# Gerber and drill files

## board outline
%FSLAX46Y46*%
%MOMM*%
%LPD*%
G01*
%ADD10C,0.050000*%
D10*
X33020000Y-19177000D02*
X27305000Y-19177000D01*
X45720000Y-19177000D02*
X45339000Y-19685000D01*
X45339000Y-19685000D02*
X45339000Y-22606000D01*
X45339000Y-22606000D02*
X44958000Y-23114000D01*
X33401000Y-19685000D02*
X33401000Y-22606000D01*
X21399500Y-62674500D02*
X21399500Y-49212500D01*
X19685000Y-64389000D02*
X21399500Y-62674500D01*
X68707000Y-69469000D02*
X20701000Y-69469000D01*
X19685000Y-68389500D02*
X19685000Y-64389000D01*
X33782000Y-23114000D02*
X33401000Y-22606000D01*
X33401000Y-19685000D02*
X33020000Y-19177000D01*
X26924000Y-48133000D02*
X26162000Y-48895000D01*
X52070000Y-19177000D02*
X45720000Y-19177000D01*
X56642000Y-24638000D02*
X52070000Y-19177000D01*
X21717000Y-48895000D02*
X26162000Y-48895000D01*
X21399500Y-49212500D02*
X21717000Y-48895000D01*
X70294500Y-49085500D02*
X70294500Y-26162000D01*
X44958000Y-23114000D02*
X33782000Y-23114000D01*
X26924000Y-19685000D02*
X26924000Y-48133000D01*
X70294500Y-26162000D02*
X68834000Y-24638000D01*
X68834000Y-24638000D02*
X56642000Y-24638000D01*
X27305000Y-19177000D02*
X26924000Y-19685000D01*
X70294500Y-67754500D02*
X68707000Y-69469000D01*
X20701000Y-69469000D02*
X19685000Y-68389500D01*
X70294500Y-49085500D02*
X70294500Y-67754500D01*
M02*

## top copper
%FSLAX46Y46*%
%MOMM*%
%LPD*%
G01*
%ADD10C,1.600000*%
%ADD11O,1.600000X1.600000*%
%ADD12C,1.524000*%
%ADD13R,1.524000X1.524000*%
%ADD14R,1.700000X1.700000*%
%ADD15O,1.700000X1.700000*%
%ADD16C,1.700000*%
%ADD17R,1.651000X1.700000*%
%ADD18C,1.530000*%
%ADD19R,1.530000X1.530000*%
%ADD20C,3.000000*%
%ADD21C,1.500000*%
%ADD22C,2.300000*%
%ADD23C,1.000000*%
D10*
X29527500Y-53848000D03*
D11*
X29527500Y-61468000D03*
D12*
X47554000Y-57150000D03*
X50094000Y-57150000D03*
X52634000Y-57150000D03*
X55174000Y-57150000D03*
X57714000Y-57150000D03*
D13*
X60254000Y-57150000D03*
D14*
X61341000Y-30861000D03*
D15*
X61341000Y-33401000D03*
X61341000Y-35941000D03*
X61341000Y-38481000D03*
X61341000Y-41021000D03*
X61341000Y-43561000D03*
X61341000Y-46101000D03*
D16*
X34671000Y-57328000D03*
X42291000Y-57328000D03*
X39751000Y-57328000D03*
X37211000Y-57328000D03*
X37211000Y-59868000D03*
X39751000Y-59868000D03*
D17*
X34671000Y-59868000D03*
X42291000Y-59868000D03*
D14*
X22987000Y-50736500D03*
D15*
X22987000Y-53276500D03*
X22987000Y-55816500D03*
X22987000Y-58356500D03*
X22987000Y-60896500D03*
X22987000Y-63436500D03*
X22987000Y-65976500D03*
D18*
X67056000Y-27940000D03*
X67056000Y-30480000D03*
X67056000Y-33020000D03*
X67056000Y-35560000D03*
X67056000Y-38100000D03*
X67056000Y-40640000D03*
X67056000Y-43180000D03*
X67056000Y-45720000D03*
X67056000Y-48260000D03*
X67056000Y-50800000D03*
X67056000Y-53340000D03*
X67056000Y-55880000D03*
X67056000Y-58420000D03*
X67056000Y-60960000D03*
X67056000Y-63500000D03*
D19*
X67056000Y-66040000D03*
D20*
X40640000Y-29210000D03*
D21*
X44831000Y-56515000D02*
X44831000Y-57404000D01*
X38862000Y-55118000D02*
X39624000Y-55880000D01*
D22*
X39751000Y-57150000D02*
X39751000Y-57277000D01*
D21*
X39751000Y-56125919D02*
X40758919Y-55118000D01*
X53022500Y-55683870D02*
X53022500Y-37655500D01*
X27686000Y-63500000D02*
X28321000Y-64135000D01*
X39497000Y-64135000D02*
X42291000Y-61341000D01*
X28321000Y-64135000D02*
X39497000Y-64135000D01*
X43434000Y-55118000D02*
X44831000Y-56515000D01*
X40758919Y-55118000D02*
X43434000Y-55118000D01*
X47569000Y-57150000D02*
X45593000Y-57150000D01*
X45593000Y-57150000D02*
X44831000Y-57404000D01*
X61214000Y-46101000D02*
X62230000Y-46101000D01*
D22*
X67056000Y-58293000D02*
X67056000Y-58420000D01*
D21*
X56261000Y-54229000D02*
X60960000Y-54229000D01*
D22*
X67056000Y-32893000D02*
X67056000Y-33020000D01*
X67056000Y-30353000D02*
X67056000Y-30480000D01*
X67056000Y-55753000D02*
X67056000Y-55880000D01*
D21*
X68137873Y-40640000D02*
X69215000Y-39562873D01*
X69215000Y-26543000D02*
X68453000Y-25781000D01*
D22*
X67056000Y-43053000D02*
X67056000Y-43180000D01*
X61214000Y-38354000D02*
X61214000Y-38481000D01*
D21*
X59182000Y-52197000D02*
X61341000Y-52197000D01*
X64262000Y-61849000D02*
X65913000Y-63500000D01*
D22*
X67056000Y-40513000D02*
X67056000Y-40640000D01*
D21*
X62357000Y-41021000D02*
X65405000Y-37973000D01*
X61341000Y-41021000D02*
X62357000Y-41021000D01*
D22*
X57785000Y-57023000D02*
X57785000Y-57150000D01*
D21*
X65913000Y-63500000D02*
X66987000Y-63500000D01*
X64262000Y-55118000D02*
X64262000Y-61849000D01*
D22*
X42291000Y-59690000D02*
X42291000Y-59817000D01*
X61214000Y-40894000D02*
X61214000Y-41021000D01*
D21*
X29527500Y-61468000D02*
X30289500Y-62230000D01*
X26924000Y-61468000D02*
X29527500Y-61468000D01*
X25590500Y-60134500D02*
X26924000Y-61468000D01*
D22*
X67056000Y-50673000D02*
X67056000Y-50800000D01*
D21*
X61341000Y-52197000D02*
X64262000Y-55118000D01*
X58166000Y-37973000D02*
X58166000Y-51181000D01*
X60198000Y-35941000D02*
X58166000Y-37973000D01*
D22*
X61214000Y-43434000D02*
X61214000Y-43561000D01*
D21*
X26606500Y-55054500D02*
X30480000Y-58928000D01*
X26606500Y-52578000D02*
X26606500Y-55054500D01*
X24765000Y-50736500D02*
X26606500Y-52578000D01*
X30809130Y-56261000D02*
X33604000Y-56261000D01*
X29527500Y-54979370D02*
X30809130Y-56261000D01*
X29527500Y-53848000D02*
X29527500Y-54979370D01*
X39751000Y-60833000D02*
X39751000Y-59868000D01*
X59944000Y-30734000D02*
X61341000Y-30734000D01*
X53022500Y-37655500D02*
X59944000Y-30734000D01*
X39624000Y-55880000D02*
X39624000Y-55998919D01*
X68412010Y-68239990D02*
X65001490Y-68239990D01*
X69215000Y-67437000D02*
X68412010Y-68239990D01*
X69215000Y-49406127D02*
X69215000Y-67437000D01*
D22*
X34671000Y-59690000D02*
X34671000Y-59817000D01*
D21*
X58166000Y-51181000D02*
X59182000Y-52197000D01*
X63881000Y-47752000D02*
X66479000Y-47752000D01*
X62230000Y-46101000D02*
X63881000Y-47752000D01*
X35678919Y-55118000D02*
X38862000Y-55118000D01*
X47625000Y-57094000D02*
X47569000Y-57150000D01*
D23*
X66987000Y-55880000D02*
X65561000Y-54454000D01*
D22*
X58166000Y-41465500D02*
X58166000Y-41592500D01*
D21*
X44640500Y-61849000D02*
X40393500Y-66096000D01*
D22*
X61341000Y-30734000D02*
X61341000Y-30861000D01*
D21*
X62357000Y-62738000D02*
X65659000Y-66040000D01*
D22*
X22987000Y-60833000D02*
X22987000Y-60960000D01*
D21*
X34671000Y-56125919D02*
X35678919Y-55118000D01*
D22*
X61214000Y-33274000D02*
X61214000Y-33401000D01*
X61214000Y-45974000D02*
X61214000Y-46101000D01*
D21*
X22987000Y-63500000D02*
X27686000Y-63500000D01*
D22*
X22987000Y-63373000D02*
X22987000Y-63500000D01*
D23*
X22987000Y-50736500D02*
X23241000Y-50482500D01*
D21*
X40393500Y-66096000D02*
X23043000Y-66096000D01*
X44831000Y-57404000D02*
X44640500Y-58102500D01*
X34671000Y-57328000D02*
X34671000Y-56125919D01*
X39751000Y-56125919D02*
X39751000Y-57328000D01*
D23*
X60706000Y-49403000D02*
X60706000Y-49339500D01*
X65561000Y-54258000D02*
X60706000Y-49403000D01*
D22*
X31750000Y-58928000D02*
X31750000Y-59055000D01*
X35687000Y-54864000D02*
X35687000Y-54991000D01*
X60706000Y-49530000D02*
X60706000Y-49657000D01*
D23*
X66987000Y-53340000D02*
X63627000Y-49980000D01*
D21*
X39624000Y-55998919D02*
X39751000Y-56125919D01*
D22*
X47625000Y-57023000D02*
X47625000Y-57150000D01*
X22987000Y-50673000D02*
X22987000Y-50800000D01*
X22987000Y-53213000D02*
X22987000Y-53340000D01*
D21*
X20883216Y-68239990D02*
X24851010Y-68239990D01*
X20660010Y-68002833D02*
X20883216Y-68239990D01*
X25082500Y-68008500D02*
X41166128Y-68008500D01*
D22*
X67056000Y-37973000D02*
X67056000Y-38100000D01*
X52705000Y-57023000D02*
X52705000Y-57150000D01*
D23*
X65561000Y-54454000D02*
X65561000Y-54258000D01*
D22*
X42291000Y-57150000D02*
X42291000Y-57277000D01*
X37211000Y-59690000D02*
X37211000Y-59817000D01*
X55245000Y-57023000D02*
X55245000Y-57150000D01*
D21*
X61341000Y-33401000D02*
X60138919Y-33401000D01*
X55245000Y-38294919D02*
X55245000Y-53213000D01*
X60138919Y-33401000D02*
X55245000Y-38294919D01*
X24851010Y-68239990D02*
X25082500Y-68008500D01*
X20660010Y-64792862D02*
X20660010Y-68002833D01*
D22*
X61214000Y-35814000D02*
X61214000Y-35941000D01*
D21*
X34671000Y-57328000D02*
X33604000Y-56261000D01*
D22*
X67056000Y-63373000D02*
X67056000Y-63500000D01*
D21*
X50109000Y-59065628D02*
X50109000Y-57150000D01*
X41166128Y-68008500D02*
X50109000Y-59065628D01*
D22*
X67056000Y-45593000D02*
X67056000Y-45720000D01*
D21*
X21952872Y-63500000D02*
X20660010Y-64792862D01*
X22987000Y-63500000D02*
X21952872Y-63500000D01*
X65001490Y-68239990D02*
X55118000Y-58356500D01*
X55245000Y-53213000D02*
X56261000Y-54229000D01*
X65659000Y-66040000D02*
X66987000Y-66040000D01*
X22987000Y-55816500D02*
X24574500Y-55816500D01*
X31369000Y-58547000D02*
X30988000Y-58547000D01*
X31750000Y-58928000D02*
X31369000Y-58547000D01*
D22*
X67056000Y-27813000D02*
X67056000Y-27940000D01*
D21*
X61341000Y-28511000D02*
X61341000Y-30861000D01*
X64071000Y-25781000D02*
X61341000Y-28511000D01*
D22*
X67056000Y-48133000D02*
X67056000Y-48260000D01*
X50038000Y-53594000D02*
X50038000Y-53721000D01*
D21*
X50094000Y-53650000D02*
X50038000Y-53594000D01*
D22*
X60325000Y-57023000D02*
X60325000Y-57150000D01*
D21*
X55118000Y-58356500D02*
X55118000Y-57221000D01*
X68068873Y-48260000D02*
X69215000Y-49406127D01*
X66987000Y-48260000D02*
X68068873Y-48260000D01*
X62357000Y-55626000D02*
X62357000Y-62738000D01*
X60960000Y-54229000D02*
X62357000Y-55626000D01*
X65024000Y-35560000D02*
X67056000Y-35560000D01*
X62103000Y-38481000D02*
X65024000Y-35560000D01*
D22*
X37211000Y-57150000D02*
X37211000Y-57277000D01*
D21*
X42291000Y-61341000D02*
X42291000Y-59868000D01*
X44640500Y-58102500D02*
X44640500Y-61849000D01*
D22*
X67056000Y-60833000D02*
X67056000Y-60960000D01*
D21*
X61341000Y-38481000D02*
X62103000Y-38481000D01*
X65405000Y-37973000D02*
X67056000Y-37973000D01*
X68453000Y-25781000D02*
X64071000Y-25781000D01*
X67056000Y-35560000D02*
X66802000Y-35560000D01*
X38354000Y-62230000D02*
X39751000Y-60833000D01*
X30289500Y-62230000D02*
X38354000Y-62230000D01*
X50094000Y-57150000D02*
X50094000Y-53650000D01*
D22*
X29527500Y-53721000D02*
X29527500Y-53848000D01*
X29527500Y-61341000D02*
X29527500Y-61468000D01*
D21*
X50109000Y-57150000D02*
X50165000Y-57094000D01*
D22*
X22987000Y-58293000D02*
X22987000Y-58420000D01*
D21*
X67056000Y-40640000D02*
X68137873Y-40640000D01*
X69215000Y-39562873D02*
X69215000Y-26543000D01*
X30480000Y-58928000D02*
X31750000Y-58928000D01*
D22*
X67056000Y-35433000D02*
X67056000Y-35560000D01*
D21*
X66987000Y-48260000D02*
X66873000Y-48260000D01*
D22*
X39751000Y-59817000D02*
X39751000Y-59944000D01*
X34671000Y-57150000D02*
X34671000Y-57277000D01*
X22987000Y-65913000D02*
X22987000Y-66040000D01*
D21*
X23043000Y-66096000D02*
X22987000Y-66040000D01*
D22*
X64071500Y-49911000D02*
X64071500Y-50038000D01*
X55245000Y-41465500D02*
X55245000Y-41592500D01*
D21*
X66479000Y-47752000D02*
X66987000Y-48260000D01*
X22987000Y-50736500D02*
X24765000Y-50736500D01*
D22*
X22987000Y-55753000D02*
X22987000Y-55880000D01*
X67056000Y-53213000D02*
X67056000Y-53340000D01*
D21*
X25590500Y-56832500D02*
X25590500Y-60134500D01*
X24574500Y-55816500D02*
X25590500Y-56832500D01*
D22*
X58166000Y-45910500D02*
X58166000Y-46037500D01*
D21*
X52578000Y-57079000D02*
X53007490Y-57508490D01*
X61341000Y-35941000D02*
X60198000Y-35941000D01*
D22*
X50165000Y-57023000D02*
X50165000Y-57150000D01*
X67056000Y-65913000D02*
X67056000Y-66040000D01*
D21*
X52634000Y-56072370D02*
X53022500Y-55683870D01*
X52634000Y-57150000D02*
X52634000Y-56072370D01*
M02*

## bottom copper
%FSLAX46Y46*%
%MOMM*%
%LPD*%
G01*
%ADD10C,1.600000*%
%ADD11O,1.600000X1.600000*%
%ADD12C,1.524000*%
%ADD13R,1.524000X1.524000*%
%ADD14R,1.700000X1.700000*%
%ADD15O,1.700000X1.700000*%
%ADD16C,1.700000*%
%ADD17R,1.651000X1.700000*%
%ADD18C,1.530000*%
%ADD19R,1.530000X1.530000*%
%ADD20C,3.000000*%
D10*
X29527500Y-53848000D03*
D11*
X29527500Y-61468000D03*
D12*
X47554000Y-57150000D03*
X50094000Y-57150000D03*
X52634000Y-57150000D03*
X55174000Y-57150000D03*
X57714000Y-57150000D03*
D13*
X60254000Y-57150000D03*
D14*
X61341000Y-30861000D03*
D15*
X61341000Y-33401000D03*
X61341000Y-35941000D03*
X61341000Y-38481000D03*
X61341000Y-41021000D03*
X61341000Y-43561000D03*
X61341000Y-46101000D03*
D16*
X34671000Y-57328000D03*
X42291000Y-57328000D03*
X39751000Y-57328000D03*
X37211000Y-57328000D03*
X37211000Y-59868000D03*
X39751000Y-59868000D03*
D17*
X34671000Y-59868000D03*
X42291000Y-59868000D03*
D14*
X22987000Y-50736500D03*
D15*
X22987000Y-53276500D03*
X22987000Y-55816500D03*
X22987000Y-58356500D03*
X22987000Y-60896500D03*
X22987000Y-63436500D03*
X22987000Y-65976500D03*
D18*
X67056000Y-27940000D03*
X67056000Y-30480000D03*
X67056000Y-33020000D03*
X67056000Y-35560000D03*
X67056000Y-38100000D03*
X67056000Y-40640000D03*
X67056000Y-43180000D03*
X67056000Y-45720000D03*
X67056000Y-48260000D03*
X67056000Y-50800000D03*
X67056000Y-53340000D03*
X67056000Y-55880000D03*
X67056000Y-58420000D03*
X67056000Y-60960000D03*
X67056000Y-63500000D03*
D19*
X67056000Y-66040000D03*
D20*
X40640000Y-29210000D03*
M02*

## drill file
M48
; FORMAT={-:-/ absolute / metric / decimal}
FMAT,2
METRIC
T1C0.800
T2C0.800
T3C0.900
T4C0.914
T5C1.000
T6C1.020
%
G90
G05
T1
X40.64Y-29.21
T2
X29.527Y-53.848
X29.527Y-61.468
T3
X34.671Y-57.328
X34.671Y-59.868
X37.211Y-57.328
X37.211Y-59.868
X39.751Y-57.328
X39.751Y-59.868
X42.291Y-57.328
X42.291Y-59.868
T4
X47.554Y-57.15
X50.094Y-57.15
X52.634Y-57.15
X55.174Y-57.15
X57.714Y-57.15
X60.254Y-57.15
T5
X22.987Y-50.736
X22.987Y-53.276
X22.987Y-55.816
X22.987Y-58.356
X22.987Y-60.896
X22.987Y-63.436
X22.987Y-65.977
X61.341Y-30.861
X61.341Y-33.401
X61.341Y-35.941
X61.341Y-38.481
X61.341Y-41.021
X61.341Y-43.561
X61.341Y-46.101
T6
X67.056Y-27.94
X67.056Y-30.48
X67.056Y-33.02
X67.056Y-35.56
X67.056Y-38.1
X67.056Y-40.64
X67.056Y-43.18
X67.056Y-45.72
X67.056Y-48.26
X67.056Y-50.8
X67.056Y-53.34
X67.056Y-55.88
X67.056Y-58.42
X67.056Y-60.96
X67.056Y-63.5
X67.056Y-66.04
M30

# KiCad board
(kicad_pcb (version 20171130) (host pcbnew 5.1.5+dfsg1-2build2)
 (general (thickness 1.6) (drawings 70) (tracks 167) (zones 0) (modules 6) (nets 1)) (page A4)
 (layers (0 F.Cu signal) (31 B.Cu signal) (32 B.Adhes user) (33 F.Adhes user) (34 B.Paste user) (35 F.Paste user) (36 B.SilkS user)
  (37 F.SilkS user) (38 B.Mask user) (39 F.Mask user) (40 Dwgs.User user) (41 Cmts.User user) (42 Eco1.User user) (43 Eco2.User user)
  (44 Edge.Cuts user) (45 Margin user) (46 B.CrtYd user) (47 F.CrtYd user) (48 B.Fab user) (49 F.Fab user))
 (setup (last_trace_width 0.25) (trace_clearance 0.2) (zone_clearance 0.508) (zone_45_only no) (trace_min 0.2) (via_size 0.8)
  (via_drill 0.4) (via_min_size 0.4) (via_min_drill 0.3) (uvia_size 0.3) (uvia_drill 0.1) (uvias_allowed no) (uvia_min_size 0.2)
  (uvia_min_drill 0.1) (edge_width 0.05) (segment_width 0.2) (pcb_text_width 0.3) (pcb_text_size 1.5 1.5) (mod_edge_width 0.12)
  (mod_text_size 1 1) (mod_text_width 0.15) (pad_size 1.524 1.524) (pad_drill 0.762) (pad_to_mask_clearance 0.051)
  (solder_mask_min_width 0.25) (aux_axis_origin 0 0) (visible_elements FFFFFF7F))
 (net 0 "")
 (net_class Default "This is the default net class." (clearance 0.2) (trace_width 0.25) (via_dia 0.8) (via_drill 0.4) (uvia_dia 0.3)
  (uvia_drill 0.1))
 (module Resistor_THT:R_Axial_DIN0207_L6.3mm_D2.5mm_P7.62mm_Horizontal (layer F.Cu) (at 29.5275 53.848 270)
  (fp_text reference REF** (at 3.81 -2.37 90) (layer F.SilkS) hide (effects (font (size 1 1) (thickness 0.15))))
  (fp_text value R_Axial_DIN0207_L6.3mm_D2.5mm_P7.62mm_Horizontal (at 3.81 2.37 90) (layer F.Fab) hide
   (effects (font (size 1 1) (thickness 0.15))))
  (pad 1 thru_hole circle (at 0 0 270) (size 1.6 1.6) (drill 0.8) (layers *.Cu *.Mask))
  (pad 2 thru_hole oval (at 7.62 0 270) (size 1.6 1.6) (drill 0.8) (layers *.Cu *.Mask)))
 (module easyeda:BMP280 (layer F.Cu) (at 53.721 61.468 270)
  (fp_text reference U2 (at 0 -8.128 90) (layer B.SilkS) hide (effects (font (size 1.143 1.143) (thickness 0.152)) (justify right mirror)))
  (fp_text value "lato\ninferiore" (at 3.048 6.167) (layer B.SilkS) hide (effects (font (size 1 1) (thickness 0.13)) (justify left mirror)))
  (pad 6 thru_hole circle (at -4.318 6.167 270) (size 1.524 1.524) (drill 0.914) (layers *.Cu *.Paste *.Mask))
  (pad 5 thru_hole circle (at -4.318 3.627) (size 1.524 1.524) (drill 0.914) (layers *.Cu *.Paste *.Mask))
  (pad 4 thru_hole circle (at -4.318 1.087) (size 1.524 1.524) (drill 0.914) (layers *.Cu *.Paste *.Mask))
  (pad 3 thru_hole circle (at -4.318 -1.453) (size 1.524 1.524) (drill 0.914) (layers *.Cu *.Paste *.Mask))
  (pad 2 thru_hole circle (at -4.318 -3.993) (size 1.524 1.524) (drill 0.914) (layers *.Cu *.Paste *.Mask))
  (pad 1 thru_hole rect (at -4.318 -6.533) (size 1.524 1.524) (drill 0.914) (layers *.Cu *.Paste *.Mask)))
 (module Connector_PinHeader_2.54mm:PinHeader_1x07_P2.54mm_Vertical (layer F.Cu) (at 61.341 30.861)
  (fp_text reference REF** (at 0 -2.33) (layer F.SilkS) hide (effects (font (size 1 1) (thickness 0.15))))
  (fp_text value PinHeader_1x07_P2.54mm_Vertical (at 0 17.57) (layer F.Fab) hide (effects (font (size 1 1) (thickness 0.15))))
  (pad 1 thru_hole rect (at 0 0) (size 1.7 1.7) (drill 1) (layers *.Cu *.Mask))
  (pad 2 thru_hole oval (at 0 2.54) (size 1.7 1.7) (drill 1) (layers *.Cu *.Mask))
  (pad 3 thru_hole oval (at 0 5.08) (size 1.7 1.7) (drill 1) (layers *.Cu *.Mask))
  (pad 4 thru_hole oval (at 0 7.62) (size 1.7 1.7) (drill 1) (layers *.Cu *.Mask))
  (pad 5 thru_hole oval (at 0 10.16) (size 1.7 1.7) (drill 1) (layers *.Cu *.Mask))
  (pad 6 thru_hole oval (at 0 12.7) (size 1.7 1.7) (drill 1) (layers *.Cu *.Mask))
  (pad 7 thru_hole oval (at 0 15.24) (size 1.7 1.7) (drill 1) (layers *.Cu *.Mask)))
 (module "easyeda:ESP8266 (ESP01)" (layer F.Cu) (at 45.466 80.518 180)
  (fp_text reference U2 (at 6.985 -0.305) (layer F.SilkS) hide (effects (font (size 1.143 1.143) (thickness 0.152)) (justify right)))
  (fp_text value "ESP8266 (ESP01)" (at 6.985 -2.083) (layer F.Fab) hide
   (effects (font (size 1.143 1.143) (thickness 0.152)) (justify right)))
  (pad VCC thru_hole circle (at 10.795 23.19 90) (size 1.7 1.7) (drill 0.9) (layers *.Cu *.Paste *.Mask))
  (pad TX thru_hole circle (at 3.175 23.19 90) (size 1.7 1.7) (drill 0.9) (layers *.Cu *.Paste *.Mask))
  (pad CH_PD thru_hole circle (at 5.715 23.19 90) (size 1.7 1.7) (drill 0.9) (layers *.Cu *.Paste *.Mask))
  (pad RST thru_hole circle (at 8.255 23.19 90) (size 1.7 1.7) (drill 0.9) (layers *.Cu *.Paste *.Mask))
  (pad GPIO0 thru_hole circle (at 8.255 20.65 90) (size 1.7 1.7) (drill 0.9) (layers *.Cu *.Paste *.Mask))
  (pad GPIO2 thru_hole circle (at 5.715 20.65 90) (size 1.7 1.7) (drill 0.9) (layers *.Cu *.Paste *.Mask))
  (pad RX thru_hole rect (at 10.795 20.65 90) (size 1.7 1.651) (drill 0.9) (layers *.Cu *.Paste *.Mask))
  (pad GND thru_hole rect (at 3.175 20.65 90) (size 1.7 1.651) (drill 0.9) (layers *.Cu *.Paste *.Mask)))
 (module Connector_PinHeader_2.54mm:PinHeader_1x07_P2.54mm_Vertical (layer F.Cu) (at 22.987 50.7365)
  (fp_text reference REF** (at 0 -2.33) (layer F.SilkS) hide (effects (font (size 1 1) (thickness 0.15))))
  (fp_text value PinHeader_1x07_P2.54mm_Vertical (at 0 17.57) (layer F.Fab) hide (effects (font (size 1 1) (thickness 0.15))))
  (pad 1 thru_hole rect (at 0 0) (size 1.7 1.7) (drill 1) (layers *.Cu *.Mask))
  (pad 2 thru_hole oval (at 0 2.54) (size 1.7 1.7) (drill 1) (layers *.Cu *.Mask))
  (pad 3 thru_hole oval (at 0 5.08) (size 1.7 1.7) (drill 1) (layers *.Cu *.Mask))
  (pad 4 thru_hole oval (at 0 7.62) (size 1.7 1.7) (drill 1) (layers *.Cu *.Mask))
  (pad 5 thru_hole oval (at 0 10.16) (size 1.7 1.7) (drill 1) (layers *.Cu *.Mask))
  (pad 6 thru_hole oval (at 0 12.7) (size 1.7 1.7) (drill 1) (layers *.Cu *.Mask))
  (pad 7 thru_hole oval (at 0 15.24) (size 1.7 1.7) (drill 1) (layers *.Cu *.Mask)))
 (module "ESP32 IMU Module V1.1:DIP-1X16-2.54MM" (layer F.Cu) (at 67.056 46.99 90)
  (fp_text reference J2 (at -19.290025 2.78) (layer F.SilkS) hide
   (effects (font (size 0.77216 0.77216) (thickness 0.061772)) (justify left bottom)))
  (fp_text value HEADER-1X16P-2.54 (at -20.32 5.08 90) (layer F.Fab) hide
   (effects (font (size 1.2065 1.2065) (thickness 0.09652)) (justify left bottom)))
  (pad 16 thru_hole circle (at 19.05 0 90) (size 1.53 1.53) (drill 1.02) (layers *.Cu *.Mask) (solder_mask_margin 0.1016))
  (pad 15 thru_hole circle (at 16.51 0 90) (size 1.53 1.53) (drill 1.02) (layers *.Cu *.Mask) (solder_mask_margin 0.1016))
  (pad 14 thru_hole circle (at 13.97 0 90) (size 1.53 1.53) (drill 1.02) (layers *.Cu *.Mask) (solder_mask_margin 0.1016))
  (pad 13 thru_hole circle (at 11.43 0 90) (size 1.53 1.53) (drill 1.02) (layers *.Cu *.Mask) (solder_mask_margin 0.1016))
  (pad 12 thru_hole circle (at 8.89 0 90) (size 1.53 1.53) (drill 1.02) (layers *.Cu *.Mask) (solder_mask_margin 0.1016))
  (pad 11 thru_hole circle (at 6.35 0 90) (size 1.53 1.53) (drill 1.02) (layers *.Cu *.Mask) (solder_mask_margin 0.1016))
  (pad 10 thru_hole circle (at 3.81 0 90) (size 1.53 1.53) (drill 1.02) (layers *.Cu *.Mask) (solder_mask_margin 0.1016))
  (pad 9 thru_hole circle (at 1.27 0 90) (size 1.53 1.53) (drill 1.02) (layers *.Cu *.Mask) (solder_mask_margin 0.1016))
  (pad 8 thru_hole circle (at -1.27 0 90) (size 1.53 1.53) (drill 1.02) (layers *.Cu *.Mask) (solder_mask_margin 0.1016))
  (pad 7 thru_hole circle (at -3.81 0 90) (size 1.53 1.53) (drill 1.02) (layers *.Cu *.Mask) (solder_mask_margin 0.1016))
  (pad 6 thru_hole circle (at -6.35 0 90) (size 1.53 1.53) (drill 1.02) (layers *.Cu *.Mask) (solder_mask_margin 0.1016))
  (pad 5 thru_hole circle (at -8.89 0 90) (size 1.53 1.53) (drill 1.02) (layers *.Cu *.Mask) (solder_mask_margin 0.1016))
  (pad 4 thru_hole circle (at -11.43 0 90) (size 1.53 1.53) (drill 1.02) (layers *.Cu *.Mask) (solder_mask_margin 0.1016))
  (pad 3 thru_hole circle (at -13.97 0 90) (size 1.53 1.53) (drill 1.02) (layers *.Cu *.Mask) (solder_mask_margin 0.1016))
  (pad 2 thru_hole circle (at -16.51 0 90) (size 1.53 1.53) (drill 1.02) (layers *.Cu *.Mask) (solder_mask_margin 0.1016))
  (pad 1 thru_hole rect (at -19.05 0 90) (size 1.53 1.53) (drill 1.02) (layers *.Cu *.Mask) (solder_mask_margin 0.1016)))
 (gr_line (start 33.02 19.177) (end 27.305 19.177) (layer Edge.Cuts) (width 0.05))
 (gr_line (start 45.72 19.177) (end 45.339 19.685) (layer Edge.Cuts) (width 0.05))
 (gr_line (start 45.339 19.685) (end 45.339 22.606) (layer Edge.Cuts) (width 0.05))
 (gr_line (start 45.339 22.606) (end 44.958 23.114) (layer Edge.Cuts) (width 0.05))
 (gr_line (start 33.401 19.685) (end 33.401 22.606) (layer Edge.Cuts) (width 0.05))
 (gr_line (start 21.3995 62.6745) (end 21.3995 49.2125) (layer Edge.Cuts) (width 0.05))
 (gr_line (start 19.685 64.389) (end 21.3995 62.6745) (layer Edge.Cuts) (width 0.05))
 (gr_line (start 68.707 69.469) (end 20.701 69.469) (layer Edge.Cuts) (width 0.05))
 (gr_line (start 19.685 68.3895) (end 19.685 64.389) (layer Edge.Cuts) (width 0.05))
 (gr_line (start 33.782 23.114) (end 33.401 22.606) (layer Edge.Cuts) (width 0.05))
 (gr_line (start 33.401 19.685) (end 33.02 19.177) (layer Edge.Cuts) (width 0.05))
 (gr_line (start 26.924 48.133) (end 26.162 48.895) (layer Edge.Cuts) (width 0.05))
 (gr_line (start 52.07 19.177) (end 45.72 19.177) (layer Edge.Cuts) (width 0.05))
 (gr_line (start 56.642 24.638) (end 52.07 19.177) (layer Edge.Cuts) (width 0.05))
 (gr_line (start 21.717 48.895) (end 26.162 48.895) (layer Edge.Cuts) (width 0.05))
 (gr_line (start 21.3995 49.2125) (end 21.717 48.895) (layer Edge.Cuts) (width 0.05))
 (gr_line (start 70.2945 49.0855) (end 70.2945 26.162) (layer Edge.Cuts) (width 0.05))
 (gr_line (start 44.958 23.114) (end 33.782 23.114) (layer Edge.Cuts) (width 0.05))
 (gr_line (start 26.924 19.685) (end 26.924 48.133) (layer Edge.Cuts) (width 0.05))
 (gr_line (start 70.2945 26.162) (end 68.834 24.638) (layer Edge.Cuts) (width 0.05))
 (gr_line (start 68.834 24.638) (end 56.642 24.638) (layer Edge.Cuts) (width 0.05))
 (gr_line (start 27.305 19.177) (end 26.924 19.685) (layer Edge.Cuts) (width 0.05))
 (gr_line (start 70.2945 67.7545) (end 68.707 69.469) (layer Edge.Cuts) (width 0.05))
 (gr_line (start 20.701 69.469) (end 19.685 68.3895) (layer Edge.Cuts) (width 0.05))
 (gr_line (start 70.2945 49.0855) (end 70.2945 67.7545) (layer Edge.Cuts) (width 0.05))
 (segment (start 44.831 56.515) (end 44.831 57.404) (width 1.5) (layer F.Cu) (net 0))
 (segment (start 38.862 55.118) (end 39.624 55.88) (width 1.5) (layer F.Cu) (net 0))
 (segment (start 39.751 57.15) (end 39.751 57.277) (width 2.3) (layer F.Cu) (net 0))
 (segment (start 39.751 56.125919) (end 40.758919 55.118) (width 1.5) (layer F.Cu) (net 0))
 (segment (start 53.0225 55.68387) (end 53.0225 37.6555) (width 1.5) (layer F.Cu) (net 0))
 (segment (start 27.686 63.5) (end 28.321 64.135) (width 1.5) (layer F.Cu) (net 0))
 (segment (start 39.497 64.135) (end 42.291 61.341) (width 1.5) (layer F.Cu) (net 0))
 (segment (start 28.321 64.135) (end 39.497 64.135) (width 1.5) (layer F.Cu) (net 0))
 (segment (start 43.434 55.118) (end 44.831 56.515) (width 1.5) (layer F.Cu) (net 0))
 (segment (start 40.758919 55.118) (end 43.434 55.118) (width 1.5) (layer F.Cu) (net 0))
 (segment (start 47.569 57.15) (end 45.593 57.15) (width 1.5) (layer F.Cu) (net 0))
 (segment (start 45.593 57.15) (end 44.831 57.404) (width 1.5) (layer F.Cu) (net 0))
 (segment (start 61.214 46.101) (end 62.23 46.101) (width 1.5) (layer F.Cu) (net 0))
 (segment (start 67.056 58.293) (end 67.056 58.42) (width 2.3) (layer F.Cu) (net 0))
 (segment (start 56.261 54.229) (end 60.96 54.229) (width 1.5) (layer F.Cu) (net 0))
 (segment (start 67.056 32.893) (end 67.056 33.02) (width 2.3) (layer F.Cu) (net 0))
 (segment (start 67.056 30.353) (end 67.056 30.48) (width 2.3) (layer F.Cu) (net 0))
 (via (at 40.64 29.21) (size 3) (drill 0.8) (layers F.Cu B.Cu) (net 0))
 (segment (start 67.056 55.753) (end 67.056 55.88) (width 2.3) (layer F.Cu) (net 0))
 (segment (start 68.137873 40.64) (end 69.215 39.562873) (width 1.5) (layer F.Cu) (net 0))
 (segment (start 69.215 26.543) (end 68.453 25.781) (width 1.5) (layer F.Cu) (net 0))
 (segment (start 67.056 43.053) (end 67.056 43.18) (width 2.3) (layer F.Cu) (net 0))
 (segment (start 61.214 38.354) (end 61.214 38.481) (width 2.3) (layer F.Cu) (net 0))
 (segment (start 59.182 52.197) (end 61.341 52.197) (width 1.5) (layer F.Cu) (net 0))
 (segment (start 64.262 61.849) (end 65.913 63.5) (width 1.5) (layer F.Cu) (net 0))
 (segment (start 67.056 40.513) (end 67.056 40.64) (width 2.3) (layer F.Cu) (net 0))
 (segment (start 62.357 41.021) (end 65.405 37.973) (width 1.5) (layer F.Cu) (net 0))
 (segment (start 61.341 41.021) (end 62.357 41.021) (width 1.5) (layer F.Cu) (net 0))
 (segment (start 57.785 57.023) (end 57.785 57.15) (width 2.3) (layer F.Cu) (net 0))
 (segment (start 65.913 63.5) (end 66.987 63.5) (width 1.5) (layer F.Cu) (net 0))
 (segment (start 64.262 55.118) (end 64.262 61.849) (width 1.5) (layer F.Cu) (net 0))
 (segment (start 42.291 59.69) (end 42.291 59.817) (width 2.3) (layer F.Cu) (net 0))
 (segment (start 61.214 40.894) (end 61.214 41.021) (width 2.3) (layer F.Cu) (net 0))
 (segment (start 29.5275 61.468) (end 30.2895 62.23) (width 1.5) (layer F.Cu) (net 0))
 (segment (start 26.924 61.468) (end 29.5275 61.468) (width 1.5) (layer F.Cu) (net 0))
 (segment (start 25.5905 60.1345) (end 26.924 61.468) (width 1.5) (layer F.Cu) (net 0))
 (segment (start 67.056 50.673) (end 67.056 50.8) (width 2.3) (layer F.Cu) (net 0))
 (segment (start 61.341 52.197) (end 64.262 55.118) (width 1.5) (layer F.Cu) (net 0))
 (segment (start 58.166 37.973) (end 58.166 51.181) (width 1.5) (layer F.Cu) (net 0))
 (segment (start 60.198 35.941) (end 58.166 37.973) (width 1.5) (layer F.Cu) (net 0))
 (segment (start 61.214 43.434) (end 61.214 43.561) (width 2.3) (layer F.Cu) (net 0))
 (segment (start 26.6065 55.0545) (end 30.48 58.928) (width 1.5) (layer F.Cu) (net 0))
 (segment (start 26.6065 52.578) (end 26.6065 55.0545) (width 1.5) (layer F.Cu) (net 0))
 (segment (start 24.765 50.7365) (end 26.6065 52.578) (width 1.5) (layer F.Cu) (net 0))
 (segment (start 30.80913 56.261) (end 33.604 56.261) (width 1.5) (layer F.Cu) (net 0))
 (segment (start 29.5275 54.97937) (end 30.80913 56.261) (width 1.5) (layer F.Cu) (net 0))
 (segment (start 29.5275 53.848) (end 29.5275 54.97937) (width 1.5) (layer F.Cu) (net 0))
 (segment (start 39.751 60.833) (end 39.751 59.868) (width 1.5) (layer F.Cu) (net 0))
 (segment (start 59.944 30.734) (end 61.341 30.734) (width 1.5) (layer F.Cu) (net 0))
 (segment (start 53.0225 37.6555) (end 59.944 30.734) (width 1.5) (layer F.Cu) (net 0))
 (segment (start 39.624 55.88) (end 39.624 55.998919) (width 1.5) (layer F.Cu) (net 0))
 (segment (start 68.41201 68.23999) (end 65.00149 68.23999) (width 1.5) (layer F.Cu) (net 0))
 (segment (start 69.215 67.437) (end 68.41201 68.23999) (width 1.5) (layer F.Cu) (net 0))
 (segment (start 69.215 49.406127) (end 69.215 67.437) (width 1.5) (layer F.Cu) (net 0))
 (segment (start 34.671 59.69) (end 34.671 59.817) (width 2.3) (layer F.Cu) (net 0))
 (segment (start 58.166 51.181) (end 59.182 52.197) (width 1.5) (layer F.Cu) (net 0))
 (segment (start 63.881 47.752) (end 66.479 47.752) (width 1.5) (layer F.Cu) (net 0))
 (segment (start 62.23 46.101) (end 63.881 47.752) (width 1.5) (layer F.Cu) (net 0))
 (segment (start 35.678919 55.118) (end 38.862 55.118) (width 1.5) (layer F.Cu) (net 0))
 (segment (start 47.625 57.094) (end 47.569 57.15) (width 1.5) (layer F.Cu) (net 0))
 (segment (start 66.987 55.88) (end 65.561 54.454) (width 1) (layer F.Cu) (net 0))
 (segment (start 58.166 41.4655) (end 58.166 41.5925) (width 2.3) (layer F.Cu) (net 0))
 (segment (start 44.6405 61.849) (end 40.3935 66.096) (width 1.5) (layer F.Cu) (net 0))
 (segment (start 61.341 30.734) (end 61.341 30.861) (width 2.3) (layer F.Cu) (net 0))
 (segment (start 62.357 62.738) (end 65.659 66.04) (width 1.5) (layer F.Cu) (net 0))
 (segment (start 22.987 60.833) (end 22.987 60.96) (width 2.3) (layer F.Cu) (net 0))
 (segment (start 34.671 56.125919) (end 35.678919 55.118) (width 1.5) (layer F.Cu) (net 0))
 (segment (start 61.214 33.274) (end 61.214 33.401) (width 2.3) (layer F.Cu) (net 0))
 (segment (start 61.214 45.974) (end 61.214 46.101) (width 2.3) (layer F.Cu) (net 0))
 (segment (start 22.987 63.5) (end 27.686 63.5) (width 1.5) (layer F.Cu) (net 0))
 (segment (start 22.987 63.373) (end 22.987 63.5) (width 2.3) (layer F.Cu) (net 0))
 (segment (start 22.987 50.7365) (end 23.241 50.4825) (width 1) (layer F.Cu) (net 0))
 (segment (start 40.3935 66.096) (end 23.043 66.096) (width 1.5) (layer F.Cu) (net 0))
 (segment (start 44.831 57.404) (end 44.6405 58.1025) (width 1.5) (layer F.Cu) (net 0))
 (segment (start 34.671 57.328) (end 34.671 56.125919) (width 1.5) (layer F.Cu) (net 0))
 (segment (start 39.751 56.125919) (end 39.751 57.328) (width 1.5) (layer F.Cu) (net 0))
 (segment (start 60.706 49.403) (end 60.706 49.3395) (width 1) (layer F.Cu) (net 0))
 (segment (start 65.561 54.258) (end 60.706 49.403) (width 1) (layer F.Cu) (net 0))
 (segment (start 31.75 58.928) (end 31.75 59.055) (width 2.3) (layer F.Cu) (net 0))
 (segment (start 35.687 54.864) (end 35.687 54.991) (width 2.3) (layer F.Cu) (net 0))
 (segment (start 60.706 49.53) (end 60.706 49.657) (width 2.3) (layer F.Cu) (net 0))
 (segment (start 66.987 53.34) (end 63.627 49.98) (width 1) (layer F.Cu) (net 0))
 (segment (start 39.624 55.998919) (end 39.751 56.125919) (width 1.5) (layer F.Cu) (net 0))
 (segment (start 47.625 57.023) (end 47.625 57.15) (width 2.3) (layer F.Cu) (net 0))
 (segment (start 22.987 50.673) (end 22.987 50.8) (width 2.3) (layer F.Cu) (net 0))
 (segment (start 22.987 53.213) (end 22.987 53.34) (width 2.3) (layer F.Cu) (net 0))
 (segment (start 20.883216 68.23999) (end 24.85101 68.23999) (width 1.5) (layer F.Cu) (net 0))
 (segment (start 20.66001 68.002833) (end 20.883216 68.23999) (width 1.5) (layer F.Cu) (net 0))
 (segment (start 25.0825 68.0085) (end 41.166128 68.0085) (width 1.5) (layer F.Cu) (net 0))
 (segment (start 67.056 37.973) (end 67.056 38.1) (width 2.3) (layer F.Cu) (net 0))
 (segment (start 52.705 57.023) (end 52.705 57.15) (width 2.3) (layer F.Cu) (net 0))
 (segment (start 65.561 54.454) (end 65.561 54.258) (width 1) (layer F.Cu) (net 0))
 (segment (start 42.291 57.15) (end 42.291 57.277) (width 2.3) (layer F.Cu) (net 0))
 (segment (start 37.211 59.69) (end 37.211 59.817) (width 2.3) (layer F.Cu) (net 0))
 (segment (start 55.245 57.023) (end 55.245 57.15) (width 2.3) (layer F.Cu) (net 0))
 (segment (start 61.341 33.401) (end 60.138919 33.401) (width 1.5) (layer F.Cu) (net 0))
 (segment (start 55.245 38.294919) (end 55.245 53.213) (width 1.5) (layer F.Cu) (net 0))
 (segment (start 60.138919 33.401) (end 55.245 38.294919) (width 1.5) (layer F.Cu) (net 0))
 (segment (start 24.85101 68.23999) (end 25.0825 68.0085) (width 1.5) (layer F.Cu) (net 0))
 (segment (start 20.66001 64.792862) (end 20.66001 68.002833) (width 1.5) (layer F.Cu) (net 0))
 (segment (start 61.214 35.814) (end 61.214 35.941) (width 2.3) (layer F.Cu) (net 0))
 (segment (start 34.671 57.328) (end 33.604 56.261) (width 1.5) (layer F.Cu) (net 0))
 (segment (start 67.056 63.373) (end 67.056 63.5) (width 2.3) (layer F.Cu) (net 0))
 (segment (start 50.109 59.065628) (end 50.109 57.15) (width 1.5) (layer F.Cu) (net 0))
 (segment (start 41.166128 68.0085) (end 50.109 59.065628) (width 1.5) (layer F.Cu) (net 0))
 (segment (start 67.056 45.593) (end 67.056 45.72) (width 2.3) (layer F.Cu) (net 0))
 (segment (start 21.952872 63.5) (end 20.66001 64.792862) (width 1.5) (layer F.Cu) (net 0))
 (segment (start 22.987 63.5) (end 21.952872 63.5) (width 1.5) (layer F.Cu) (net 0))
 (segment (start 65.00149 68.23999) (end 55.118 58.3565) (width 1.5) (layer F.Cu) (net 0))
 (segment (start 55.245 53.213) (end 56.261 54.229) (width 1.5) (layer F.Cu) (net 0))
 (segment (start 65.659 66.04) (end 66.987 66.04) (width 1.5) (layer F.Cu) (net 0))
 (segment (start 22.987 55.8165) (end 24.5745 55.8165) (width 1.5) (layer F.Cu) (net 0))
 (segment (start 31.369 58.547) (end 30.988 58.547) (width 1.5) (layer F.Cu) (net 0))
 (segment (start 31.75 58.928) (end 31.369 58.547) (width 1.5) (layer F.Cu) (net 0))
 (segment (start 67.056 27.813) (end 67.056 27.94) (width 2.3) (layer F.Cu) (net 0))
 (segment (start 61.341 28.511) (end 61.341 30.861) (width 1.5) (layer F.Cu) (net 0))
 (segment (start 64.071 25.781) (end 61.341 28.511) (width 1.5) (layer F.Cu) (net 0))
 (segment (start 67.056 48.133) (end 67.056 48.26) (width 2.3) (layer F.Cu) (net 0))
 (segment (start 50.038 53.594) (end 50.038 53.721) (width 2.3) (layer F.Cu) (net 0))
 (segment (start 50.094 53.65) (end 50.038 53.594) (width 1.5) (layer F.Cu) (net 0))
 (segment (start 60.325 57.023) (end 60.325 57.15) (width 2.3) (layer F.Cu) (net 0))
 (segment (start 55.118 58.3565) (end 55.118 57.221) (width 1.5) (layer F.Cu) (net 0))
 (segment (start 68.068873 48.26) (end 69.215 49.406127) (width 1.5) (layer F.Cu) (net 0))
 (segment (start 66.987 48.26) (end 68.068873 48.26) (width 1.5) (layer F.Cu) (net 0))
 (segment (start 62.357 55.626) (end 62.357 62.738) (width 1.5) (layer F.Cu) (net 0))
 (segment (start 60.96 54.229) (end 62.357 55.626) (width 1.5) (layer F.Cu) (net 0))
 (segment (start 65.024 35.56) (end 67.056 35.56) (width 1.5) (layer F.Cu) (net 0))
 (segment (start 62.103 38.481) (end 65.024 35.56) (width 1.5) (layer F.Cu) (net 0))
 (segment (start 37.211 57.15) (end 37.211 57.277) (width 2.3) (layer F.Cu) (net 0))
 (segment (start 42.291 61.341) (end 42.291 59.868) (width 1.5) (layer F.Cu) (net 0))
 (segment (start 44.6405 58.1025) (end 44.6405 61.849) (width 1.5) (layer F.Cu) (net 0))
 (segment (start 67.056 60.833) (end 67.056 60.96) (width 2.3) (layer F.Cu) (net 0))
 (segment (start 61.341 38.481) (end 62.103 38.481) (width 1.5) (layer F.Cu) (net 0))
 (segment (start 65.405 37.973) (end 67.056 37.973) (width 1.5) (layer F.Cu) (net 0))
 (segment (start 68.453 25.781) (end 64.071 25.781) (width 1.5) (layer F.Cu) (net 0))
 (segment (start 67.056 35.56) (end 66.802 35.56) (width 1.5) (layer F.Cu) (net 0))
 (segment (start 38.354 62.23) (end 39.751 60.833) (width 1.5) (layer F.Cu) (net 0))
 (segment (start 30.2895 62.23) (end 38.354 62.23) (width 1.5) (layer F.Cu) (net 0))
 (segment (start 50.094 57.15) (end 50.094 53.65) (width 1.5) (layer F.Cu) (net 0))
 (segment (start 29.5275 53.721) (end 29.5275 53.848) (width 2.3) (layer F.Cu) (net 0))
 (segment (start 29.5275 61.341) (end 29.5275 61.468) (width 2.3) (layer F.Cu) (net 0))
 (segment (start 50.109 57.15) (end 50.165 57.094) (width 1.5) (layer F.Cu) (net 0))
 (segment (start 22.987 58.293) (end 22.987 58.42) (width 2.3) (layer F.Cu) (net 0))
 (segment (start 67.056 40.64) (end 68.137873 40.64) (width 1.5) (layer F.Cu) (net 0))
 (segment (start 69.215 39.562873) (end 69.215 26.543) (width 1.5) (layer F.Cu) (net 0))
 (segment (start 30.48 58.928) (end 31.75 58.928) (width 1.5) (layer F.Cu) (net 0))
 (segment (start 67.056 35.433) (end 67.056 35.56) (width 2.3) (layer F.Cu) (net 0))
 (segment (start 66.987 48.26) (end 66.873 48.26) (width 1.5) (layer F.Cu) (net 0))
 (segment (start 39.751 59.817) (end 39.751 59.944) (width 2.3) (layer F.Cu) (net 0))
 (segment (start 34.671 57.15) (end 34.671 57.277) (width 2.3) (layer F.Cu) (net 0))
 (segment (start 22.987 65.913) (end 22.987 66.04) (width 2.3) (layer F.Cu) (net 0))
 (segment (start 23.043 66.096) (end 22.987 66.04) (width 1.5) (layer F.Cu) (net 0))
 (segment (start 64.0715 49.911) (end 64.0715 50.038) (width 2.3) (layer F.Cu) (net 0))
 (segment (start 55.245 41.4655) (end 55.245 41.5925) (width 2.3) (layer F.Cu) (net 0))
 (segment (start 66.479 47.752) (end 66.987 48.26) (width 1.5) (layer F.Cu) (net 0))
 (segment (start 22.987 50.7365) (end 24.765 50.7365) (width 1.5) (layer F.Cu) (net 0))
 (segment (start 22.987 55.753) (end 22.987 55.88) (width 2.3) (layer F.Cu) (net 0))
 (segment (start 67.056 53.213) (end 67.056 53.34) (width 2.3) (layer F.Cu) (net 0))
 (segment (start 25.5905 56.8325) (end 25.5905 60.1345) (width 1.5) (layer F.Cu) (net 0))
 (segment (start 24.5745 55.8165) (end 25.5905 56.8325) (width 1.5) (layer F.Cu) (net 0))
 (segment (start 58.166 45.9105) (end 58.166 46.0375) (width 2.3) (layer F.Cu) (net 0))
 (segment (start 52.578 57.079) (end 53.00749 57.50849) (width 1.5) (layer F.Cu) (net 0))
 (segment (start 61.341 35.941) (end 60.198 35.941) (width 1.5) (layer F.Cu) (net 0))
 (segment (start 50.165 57.023) (end 50.165 57.15) (width 2.3) (layer F.Cu) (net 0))
 (segment (start 67.056 65.913) (end 67.056 66.04) (width 2.3) (layer F.Cu) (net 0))
 (segment (start 52.634 56.07237) (end 53.0225 55.68387) (width 1.5) (layer F.Cu) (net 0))
 (segment (start 52.634 57.15) (end 52.634 56.07237) (width 1.5) (layer F.Cu) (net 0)))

